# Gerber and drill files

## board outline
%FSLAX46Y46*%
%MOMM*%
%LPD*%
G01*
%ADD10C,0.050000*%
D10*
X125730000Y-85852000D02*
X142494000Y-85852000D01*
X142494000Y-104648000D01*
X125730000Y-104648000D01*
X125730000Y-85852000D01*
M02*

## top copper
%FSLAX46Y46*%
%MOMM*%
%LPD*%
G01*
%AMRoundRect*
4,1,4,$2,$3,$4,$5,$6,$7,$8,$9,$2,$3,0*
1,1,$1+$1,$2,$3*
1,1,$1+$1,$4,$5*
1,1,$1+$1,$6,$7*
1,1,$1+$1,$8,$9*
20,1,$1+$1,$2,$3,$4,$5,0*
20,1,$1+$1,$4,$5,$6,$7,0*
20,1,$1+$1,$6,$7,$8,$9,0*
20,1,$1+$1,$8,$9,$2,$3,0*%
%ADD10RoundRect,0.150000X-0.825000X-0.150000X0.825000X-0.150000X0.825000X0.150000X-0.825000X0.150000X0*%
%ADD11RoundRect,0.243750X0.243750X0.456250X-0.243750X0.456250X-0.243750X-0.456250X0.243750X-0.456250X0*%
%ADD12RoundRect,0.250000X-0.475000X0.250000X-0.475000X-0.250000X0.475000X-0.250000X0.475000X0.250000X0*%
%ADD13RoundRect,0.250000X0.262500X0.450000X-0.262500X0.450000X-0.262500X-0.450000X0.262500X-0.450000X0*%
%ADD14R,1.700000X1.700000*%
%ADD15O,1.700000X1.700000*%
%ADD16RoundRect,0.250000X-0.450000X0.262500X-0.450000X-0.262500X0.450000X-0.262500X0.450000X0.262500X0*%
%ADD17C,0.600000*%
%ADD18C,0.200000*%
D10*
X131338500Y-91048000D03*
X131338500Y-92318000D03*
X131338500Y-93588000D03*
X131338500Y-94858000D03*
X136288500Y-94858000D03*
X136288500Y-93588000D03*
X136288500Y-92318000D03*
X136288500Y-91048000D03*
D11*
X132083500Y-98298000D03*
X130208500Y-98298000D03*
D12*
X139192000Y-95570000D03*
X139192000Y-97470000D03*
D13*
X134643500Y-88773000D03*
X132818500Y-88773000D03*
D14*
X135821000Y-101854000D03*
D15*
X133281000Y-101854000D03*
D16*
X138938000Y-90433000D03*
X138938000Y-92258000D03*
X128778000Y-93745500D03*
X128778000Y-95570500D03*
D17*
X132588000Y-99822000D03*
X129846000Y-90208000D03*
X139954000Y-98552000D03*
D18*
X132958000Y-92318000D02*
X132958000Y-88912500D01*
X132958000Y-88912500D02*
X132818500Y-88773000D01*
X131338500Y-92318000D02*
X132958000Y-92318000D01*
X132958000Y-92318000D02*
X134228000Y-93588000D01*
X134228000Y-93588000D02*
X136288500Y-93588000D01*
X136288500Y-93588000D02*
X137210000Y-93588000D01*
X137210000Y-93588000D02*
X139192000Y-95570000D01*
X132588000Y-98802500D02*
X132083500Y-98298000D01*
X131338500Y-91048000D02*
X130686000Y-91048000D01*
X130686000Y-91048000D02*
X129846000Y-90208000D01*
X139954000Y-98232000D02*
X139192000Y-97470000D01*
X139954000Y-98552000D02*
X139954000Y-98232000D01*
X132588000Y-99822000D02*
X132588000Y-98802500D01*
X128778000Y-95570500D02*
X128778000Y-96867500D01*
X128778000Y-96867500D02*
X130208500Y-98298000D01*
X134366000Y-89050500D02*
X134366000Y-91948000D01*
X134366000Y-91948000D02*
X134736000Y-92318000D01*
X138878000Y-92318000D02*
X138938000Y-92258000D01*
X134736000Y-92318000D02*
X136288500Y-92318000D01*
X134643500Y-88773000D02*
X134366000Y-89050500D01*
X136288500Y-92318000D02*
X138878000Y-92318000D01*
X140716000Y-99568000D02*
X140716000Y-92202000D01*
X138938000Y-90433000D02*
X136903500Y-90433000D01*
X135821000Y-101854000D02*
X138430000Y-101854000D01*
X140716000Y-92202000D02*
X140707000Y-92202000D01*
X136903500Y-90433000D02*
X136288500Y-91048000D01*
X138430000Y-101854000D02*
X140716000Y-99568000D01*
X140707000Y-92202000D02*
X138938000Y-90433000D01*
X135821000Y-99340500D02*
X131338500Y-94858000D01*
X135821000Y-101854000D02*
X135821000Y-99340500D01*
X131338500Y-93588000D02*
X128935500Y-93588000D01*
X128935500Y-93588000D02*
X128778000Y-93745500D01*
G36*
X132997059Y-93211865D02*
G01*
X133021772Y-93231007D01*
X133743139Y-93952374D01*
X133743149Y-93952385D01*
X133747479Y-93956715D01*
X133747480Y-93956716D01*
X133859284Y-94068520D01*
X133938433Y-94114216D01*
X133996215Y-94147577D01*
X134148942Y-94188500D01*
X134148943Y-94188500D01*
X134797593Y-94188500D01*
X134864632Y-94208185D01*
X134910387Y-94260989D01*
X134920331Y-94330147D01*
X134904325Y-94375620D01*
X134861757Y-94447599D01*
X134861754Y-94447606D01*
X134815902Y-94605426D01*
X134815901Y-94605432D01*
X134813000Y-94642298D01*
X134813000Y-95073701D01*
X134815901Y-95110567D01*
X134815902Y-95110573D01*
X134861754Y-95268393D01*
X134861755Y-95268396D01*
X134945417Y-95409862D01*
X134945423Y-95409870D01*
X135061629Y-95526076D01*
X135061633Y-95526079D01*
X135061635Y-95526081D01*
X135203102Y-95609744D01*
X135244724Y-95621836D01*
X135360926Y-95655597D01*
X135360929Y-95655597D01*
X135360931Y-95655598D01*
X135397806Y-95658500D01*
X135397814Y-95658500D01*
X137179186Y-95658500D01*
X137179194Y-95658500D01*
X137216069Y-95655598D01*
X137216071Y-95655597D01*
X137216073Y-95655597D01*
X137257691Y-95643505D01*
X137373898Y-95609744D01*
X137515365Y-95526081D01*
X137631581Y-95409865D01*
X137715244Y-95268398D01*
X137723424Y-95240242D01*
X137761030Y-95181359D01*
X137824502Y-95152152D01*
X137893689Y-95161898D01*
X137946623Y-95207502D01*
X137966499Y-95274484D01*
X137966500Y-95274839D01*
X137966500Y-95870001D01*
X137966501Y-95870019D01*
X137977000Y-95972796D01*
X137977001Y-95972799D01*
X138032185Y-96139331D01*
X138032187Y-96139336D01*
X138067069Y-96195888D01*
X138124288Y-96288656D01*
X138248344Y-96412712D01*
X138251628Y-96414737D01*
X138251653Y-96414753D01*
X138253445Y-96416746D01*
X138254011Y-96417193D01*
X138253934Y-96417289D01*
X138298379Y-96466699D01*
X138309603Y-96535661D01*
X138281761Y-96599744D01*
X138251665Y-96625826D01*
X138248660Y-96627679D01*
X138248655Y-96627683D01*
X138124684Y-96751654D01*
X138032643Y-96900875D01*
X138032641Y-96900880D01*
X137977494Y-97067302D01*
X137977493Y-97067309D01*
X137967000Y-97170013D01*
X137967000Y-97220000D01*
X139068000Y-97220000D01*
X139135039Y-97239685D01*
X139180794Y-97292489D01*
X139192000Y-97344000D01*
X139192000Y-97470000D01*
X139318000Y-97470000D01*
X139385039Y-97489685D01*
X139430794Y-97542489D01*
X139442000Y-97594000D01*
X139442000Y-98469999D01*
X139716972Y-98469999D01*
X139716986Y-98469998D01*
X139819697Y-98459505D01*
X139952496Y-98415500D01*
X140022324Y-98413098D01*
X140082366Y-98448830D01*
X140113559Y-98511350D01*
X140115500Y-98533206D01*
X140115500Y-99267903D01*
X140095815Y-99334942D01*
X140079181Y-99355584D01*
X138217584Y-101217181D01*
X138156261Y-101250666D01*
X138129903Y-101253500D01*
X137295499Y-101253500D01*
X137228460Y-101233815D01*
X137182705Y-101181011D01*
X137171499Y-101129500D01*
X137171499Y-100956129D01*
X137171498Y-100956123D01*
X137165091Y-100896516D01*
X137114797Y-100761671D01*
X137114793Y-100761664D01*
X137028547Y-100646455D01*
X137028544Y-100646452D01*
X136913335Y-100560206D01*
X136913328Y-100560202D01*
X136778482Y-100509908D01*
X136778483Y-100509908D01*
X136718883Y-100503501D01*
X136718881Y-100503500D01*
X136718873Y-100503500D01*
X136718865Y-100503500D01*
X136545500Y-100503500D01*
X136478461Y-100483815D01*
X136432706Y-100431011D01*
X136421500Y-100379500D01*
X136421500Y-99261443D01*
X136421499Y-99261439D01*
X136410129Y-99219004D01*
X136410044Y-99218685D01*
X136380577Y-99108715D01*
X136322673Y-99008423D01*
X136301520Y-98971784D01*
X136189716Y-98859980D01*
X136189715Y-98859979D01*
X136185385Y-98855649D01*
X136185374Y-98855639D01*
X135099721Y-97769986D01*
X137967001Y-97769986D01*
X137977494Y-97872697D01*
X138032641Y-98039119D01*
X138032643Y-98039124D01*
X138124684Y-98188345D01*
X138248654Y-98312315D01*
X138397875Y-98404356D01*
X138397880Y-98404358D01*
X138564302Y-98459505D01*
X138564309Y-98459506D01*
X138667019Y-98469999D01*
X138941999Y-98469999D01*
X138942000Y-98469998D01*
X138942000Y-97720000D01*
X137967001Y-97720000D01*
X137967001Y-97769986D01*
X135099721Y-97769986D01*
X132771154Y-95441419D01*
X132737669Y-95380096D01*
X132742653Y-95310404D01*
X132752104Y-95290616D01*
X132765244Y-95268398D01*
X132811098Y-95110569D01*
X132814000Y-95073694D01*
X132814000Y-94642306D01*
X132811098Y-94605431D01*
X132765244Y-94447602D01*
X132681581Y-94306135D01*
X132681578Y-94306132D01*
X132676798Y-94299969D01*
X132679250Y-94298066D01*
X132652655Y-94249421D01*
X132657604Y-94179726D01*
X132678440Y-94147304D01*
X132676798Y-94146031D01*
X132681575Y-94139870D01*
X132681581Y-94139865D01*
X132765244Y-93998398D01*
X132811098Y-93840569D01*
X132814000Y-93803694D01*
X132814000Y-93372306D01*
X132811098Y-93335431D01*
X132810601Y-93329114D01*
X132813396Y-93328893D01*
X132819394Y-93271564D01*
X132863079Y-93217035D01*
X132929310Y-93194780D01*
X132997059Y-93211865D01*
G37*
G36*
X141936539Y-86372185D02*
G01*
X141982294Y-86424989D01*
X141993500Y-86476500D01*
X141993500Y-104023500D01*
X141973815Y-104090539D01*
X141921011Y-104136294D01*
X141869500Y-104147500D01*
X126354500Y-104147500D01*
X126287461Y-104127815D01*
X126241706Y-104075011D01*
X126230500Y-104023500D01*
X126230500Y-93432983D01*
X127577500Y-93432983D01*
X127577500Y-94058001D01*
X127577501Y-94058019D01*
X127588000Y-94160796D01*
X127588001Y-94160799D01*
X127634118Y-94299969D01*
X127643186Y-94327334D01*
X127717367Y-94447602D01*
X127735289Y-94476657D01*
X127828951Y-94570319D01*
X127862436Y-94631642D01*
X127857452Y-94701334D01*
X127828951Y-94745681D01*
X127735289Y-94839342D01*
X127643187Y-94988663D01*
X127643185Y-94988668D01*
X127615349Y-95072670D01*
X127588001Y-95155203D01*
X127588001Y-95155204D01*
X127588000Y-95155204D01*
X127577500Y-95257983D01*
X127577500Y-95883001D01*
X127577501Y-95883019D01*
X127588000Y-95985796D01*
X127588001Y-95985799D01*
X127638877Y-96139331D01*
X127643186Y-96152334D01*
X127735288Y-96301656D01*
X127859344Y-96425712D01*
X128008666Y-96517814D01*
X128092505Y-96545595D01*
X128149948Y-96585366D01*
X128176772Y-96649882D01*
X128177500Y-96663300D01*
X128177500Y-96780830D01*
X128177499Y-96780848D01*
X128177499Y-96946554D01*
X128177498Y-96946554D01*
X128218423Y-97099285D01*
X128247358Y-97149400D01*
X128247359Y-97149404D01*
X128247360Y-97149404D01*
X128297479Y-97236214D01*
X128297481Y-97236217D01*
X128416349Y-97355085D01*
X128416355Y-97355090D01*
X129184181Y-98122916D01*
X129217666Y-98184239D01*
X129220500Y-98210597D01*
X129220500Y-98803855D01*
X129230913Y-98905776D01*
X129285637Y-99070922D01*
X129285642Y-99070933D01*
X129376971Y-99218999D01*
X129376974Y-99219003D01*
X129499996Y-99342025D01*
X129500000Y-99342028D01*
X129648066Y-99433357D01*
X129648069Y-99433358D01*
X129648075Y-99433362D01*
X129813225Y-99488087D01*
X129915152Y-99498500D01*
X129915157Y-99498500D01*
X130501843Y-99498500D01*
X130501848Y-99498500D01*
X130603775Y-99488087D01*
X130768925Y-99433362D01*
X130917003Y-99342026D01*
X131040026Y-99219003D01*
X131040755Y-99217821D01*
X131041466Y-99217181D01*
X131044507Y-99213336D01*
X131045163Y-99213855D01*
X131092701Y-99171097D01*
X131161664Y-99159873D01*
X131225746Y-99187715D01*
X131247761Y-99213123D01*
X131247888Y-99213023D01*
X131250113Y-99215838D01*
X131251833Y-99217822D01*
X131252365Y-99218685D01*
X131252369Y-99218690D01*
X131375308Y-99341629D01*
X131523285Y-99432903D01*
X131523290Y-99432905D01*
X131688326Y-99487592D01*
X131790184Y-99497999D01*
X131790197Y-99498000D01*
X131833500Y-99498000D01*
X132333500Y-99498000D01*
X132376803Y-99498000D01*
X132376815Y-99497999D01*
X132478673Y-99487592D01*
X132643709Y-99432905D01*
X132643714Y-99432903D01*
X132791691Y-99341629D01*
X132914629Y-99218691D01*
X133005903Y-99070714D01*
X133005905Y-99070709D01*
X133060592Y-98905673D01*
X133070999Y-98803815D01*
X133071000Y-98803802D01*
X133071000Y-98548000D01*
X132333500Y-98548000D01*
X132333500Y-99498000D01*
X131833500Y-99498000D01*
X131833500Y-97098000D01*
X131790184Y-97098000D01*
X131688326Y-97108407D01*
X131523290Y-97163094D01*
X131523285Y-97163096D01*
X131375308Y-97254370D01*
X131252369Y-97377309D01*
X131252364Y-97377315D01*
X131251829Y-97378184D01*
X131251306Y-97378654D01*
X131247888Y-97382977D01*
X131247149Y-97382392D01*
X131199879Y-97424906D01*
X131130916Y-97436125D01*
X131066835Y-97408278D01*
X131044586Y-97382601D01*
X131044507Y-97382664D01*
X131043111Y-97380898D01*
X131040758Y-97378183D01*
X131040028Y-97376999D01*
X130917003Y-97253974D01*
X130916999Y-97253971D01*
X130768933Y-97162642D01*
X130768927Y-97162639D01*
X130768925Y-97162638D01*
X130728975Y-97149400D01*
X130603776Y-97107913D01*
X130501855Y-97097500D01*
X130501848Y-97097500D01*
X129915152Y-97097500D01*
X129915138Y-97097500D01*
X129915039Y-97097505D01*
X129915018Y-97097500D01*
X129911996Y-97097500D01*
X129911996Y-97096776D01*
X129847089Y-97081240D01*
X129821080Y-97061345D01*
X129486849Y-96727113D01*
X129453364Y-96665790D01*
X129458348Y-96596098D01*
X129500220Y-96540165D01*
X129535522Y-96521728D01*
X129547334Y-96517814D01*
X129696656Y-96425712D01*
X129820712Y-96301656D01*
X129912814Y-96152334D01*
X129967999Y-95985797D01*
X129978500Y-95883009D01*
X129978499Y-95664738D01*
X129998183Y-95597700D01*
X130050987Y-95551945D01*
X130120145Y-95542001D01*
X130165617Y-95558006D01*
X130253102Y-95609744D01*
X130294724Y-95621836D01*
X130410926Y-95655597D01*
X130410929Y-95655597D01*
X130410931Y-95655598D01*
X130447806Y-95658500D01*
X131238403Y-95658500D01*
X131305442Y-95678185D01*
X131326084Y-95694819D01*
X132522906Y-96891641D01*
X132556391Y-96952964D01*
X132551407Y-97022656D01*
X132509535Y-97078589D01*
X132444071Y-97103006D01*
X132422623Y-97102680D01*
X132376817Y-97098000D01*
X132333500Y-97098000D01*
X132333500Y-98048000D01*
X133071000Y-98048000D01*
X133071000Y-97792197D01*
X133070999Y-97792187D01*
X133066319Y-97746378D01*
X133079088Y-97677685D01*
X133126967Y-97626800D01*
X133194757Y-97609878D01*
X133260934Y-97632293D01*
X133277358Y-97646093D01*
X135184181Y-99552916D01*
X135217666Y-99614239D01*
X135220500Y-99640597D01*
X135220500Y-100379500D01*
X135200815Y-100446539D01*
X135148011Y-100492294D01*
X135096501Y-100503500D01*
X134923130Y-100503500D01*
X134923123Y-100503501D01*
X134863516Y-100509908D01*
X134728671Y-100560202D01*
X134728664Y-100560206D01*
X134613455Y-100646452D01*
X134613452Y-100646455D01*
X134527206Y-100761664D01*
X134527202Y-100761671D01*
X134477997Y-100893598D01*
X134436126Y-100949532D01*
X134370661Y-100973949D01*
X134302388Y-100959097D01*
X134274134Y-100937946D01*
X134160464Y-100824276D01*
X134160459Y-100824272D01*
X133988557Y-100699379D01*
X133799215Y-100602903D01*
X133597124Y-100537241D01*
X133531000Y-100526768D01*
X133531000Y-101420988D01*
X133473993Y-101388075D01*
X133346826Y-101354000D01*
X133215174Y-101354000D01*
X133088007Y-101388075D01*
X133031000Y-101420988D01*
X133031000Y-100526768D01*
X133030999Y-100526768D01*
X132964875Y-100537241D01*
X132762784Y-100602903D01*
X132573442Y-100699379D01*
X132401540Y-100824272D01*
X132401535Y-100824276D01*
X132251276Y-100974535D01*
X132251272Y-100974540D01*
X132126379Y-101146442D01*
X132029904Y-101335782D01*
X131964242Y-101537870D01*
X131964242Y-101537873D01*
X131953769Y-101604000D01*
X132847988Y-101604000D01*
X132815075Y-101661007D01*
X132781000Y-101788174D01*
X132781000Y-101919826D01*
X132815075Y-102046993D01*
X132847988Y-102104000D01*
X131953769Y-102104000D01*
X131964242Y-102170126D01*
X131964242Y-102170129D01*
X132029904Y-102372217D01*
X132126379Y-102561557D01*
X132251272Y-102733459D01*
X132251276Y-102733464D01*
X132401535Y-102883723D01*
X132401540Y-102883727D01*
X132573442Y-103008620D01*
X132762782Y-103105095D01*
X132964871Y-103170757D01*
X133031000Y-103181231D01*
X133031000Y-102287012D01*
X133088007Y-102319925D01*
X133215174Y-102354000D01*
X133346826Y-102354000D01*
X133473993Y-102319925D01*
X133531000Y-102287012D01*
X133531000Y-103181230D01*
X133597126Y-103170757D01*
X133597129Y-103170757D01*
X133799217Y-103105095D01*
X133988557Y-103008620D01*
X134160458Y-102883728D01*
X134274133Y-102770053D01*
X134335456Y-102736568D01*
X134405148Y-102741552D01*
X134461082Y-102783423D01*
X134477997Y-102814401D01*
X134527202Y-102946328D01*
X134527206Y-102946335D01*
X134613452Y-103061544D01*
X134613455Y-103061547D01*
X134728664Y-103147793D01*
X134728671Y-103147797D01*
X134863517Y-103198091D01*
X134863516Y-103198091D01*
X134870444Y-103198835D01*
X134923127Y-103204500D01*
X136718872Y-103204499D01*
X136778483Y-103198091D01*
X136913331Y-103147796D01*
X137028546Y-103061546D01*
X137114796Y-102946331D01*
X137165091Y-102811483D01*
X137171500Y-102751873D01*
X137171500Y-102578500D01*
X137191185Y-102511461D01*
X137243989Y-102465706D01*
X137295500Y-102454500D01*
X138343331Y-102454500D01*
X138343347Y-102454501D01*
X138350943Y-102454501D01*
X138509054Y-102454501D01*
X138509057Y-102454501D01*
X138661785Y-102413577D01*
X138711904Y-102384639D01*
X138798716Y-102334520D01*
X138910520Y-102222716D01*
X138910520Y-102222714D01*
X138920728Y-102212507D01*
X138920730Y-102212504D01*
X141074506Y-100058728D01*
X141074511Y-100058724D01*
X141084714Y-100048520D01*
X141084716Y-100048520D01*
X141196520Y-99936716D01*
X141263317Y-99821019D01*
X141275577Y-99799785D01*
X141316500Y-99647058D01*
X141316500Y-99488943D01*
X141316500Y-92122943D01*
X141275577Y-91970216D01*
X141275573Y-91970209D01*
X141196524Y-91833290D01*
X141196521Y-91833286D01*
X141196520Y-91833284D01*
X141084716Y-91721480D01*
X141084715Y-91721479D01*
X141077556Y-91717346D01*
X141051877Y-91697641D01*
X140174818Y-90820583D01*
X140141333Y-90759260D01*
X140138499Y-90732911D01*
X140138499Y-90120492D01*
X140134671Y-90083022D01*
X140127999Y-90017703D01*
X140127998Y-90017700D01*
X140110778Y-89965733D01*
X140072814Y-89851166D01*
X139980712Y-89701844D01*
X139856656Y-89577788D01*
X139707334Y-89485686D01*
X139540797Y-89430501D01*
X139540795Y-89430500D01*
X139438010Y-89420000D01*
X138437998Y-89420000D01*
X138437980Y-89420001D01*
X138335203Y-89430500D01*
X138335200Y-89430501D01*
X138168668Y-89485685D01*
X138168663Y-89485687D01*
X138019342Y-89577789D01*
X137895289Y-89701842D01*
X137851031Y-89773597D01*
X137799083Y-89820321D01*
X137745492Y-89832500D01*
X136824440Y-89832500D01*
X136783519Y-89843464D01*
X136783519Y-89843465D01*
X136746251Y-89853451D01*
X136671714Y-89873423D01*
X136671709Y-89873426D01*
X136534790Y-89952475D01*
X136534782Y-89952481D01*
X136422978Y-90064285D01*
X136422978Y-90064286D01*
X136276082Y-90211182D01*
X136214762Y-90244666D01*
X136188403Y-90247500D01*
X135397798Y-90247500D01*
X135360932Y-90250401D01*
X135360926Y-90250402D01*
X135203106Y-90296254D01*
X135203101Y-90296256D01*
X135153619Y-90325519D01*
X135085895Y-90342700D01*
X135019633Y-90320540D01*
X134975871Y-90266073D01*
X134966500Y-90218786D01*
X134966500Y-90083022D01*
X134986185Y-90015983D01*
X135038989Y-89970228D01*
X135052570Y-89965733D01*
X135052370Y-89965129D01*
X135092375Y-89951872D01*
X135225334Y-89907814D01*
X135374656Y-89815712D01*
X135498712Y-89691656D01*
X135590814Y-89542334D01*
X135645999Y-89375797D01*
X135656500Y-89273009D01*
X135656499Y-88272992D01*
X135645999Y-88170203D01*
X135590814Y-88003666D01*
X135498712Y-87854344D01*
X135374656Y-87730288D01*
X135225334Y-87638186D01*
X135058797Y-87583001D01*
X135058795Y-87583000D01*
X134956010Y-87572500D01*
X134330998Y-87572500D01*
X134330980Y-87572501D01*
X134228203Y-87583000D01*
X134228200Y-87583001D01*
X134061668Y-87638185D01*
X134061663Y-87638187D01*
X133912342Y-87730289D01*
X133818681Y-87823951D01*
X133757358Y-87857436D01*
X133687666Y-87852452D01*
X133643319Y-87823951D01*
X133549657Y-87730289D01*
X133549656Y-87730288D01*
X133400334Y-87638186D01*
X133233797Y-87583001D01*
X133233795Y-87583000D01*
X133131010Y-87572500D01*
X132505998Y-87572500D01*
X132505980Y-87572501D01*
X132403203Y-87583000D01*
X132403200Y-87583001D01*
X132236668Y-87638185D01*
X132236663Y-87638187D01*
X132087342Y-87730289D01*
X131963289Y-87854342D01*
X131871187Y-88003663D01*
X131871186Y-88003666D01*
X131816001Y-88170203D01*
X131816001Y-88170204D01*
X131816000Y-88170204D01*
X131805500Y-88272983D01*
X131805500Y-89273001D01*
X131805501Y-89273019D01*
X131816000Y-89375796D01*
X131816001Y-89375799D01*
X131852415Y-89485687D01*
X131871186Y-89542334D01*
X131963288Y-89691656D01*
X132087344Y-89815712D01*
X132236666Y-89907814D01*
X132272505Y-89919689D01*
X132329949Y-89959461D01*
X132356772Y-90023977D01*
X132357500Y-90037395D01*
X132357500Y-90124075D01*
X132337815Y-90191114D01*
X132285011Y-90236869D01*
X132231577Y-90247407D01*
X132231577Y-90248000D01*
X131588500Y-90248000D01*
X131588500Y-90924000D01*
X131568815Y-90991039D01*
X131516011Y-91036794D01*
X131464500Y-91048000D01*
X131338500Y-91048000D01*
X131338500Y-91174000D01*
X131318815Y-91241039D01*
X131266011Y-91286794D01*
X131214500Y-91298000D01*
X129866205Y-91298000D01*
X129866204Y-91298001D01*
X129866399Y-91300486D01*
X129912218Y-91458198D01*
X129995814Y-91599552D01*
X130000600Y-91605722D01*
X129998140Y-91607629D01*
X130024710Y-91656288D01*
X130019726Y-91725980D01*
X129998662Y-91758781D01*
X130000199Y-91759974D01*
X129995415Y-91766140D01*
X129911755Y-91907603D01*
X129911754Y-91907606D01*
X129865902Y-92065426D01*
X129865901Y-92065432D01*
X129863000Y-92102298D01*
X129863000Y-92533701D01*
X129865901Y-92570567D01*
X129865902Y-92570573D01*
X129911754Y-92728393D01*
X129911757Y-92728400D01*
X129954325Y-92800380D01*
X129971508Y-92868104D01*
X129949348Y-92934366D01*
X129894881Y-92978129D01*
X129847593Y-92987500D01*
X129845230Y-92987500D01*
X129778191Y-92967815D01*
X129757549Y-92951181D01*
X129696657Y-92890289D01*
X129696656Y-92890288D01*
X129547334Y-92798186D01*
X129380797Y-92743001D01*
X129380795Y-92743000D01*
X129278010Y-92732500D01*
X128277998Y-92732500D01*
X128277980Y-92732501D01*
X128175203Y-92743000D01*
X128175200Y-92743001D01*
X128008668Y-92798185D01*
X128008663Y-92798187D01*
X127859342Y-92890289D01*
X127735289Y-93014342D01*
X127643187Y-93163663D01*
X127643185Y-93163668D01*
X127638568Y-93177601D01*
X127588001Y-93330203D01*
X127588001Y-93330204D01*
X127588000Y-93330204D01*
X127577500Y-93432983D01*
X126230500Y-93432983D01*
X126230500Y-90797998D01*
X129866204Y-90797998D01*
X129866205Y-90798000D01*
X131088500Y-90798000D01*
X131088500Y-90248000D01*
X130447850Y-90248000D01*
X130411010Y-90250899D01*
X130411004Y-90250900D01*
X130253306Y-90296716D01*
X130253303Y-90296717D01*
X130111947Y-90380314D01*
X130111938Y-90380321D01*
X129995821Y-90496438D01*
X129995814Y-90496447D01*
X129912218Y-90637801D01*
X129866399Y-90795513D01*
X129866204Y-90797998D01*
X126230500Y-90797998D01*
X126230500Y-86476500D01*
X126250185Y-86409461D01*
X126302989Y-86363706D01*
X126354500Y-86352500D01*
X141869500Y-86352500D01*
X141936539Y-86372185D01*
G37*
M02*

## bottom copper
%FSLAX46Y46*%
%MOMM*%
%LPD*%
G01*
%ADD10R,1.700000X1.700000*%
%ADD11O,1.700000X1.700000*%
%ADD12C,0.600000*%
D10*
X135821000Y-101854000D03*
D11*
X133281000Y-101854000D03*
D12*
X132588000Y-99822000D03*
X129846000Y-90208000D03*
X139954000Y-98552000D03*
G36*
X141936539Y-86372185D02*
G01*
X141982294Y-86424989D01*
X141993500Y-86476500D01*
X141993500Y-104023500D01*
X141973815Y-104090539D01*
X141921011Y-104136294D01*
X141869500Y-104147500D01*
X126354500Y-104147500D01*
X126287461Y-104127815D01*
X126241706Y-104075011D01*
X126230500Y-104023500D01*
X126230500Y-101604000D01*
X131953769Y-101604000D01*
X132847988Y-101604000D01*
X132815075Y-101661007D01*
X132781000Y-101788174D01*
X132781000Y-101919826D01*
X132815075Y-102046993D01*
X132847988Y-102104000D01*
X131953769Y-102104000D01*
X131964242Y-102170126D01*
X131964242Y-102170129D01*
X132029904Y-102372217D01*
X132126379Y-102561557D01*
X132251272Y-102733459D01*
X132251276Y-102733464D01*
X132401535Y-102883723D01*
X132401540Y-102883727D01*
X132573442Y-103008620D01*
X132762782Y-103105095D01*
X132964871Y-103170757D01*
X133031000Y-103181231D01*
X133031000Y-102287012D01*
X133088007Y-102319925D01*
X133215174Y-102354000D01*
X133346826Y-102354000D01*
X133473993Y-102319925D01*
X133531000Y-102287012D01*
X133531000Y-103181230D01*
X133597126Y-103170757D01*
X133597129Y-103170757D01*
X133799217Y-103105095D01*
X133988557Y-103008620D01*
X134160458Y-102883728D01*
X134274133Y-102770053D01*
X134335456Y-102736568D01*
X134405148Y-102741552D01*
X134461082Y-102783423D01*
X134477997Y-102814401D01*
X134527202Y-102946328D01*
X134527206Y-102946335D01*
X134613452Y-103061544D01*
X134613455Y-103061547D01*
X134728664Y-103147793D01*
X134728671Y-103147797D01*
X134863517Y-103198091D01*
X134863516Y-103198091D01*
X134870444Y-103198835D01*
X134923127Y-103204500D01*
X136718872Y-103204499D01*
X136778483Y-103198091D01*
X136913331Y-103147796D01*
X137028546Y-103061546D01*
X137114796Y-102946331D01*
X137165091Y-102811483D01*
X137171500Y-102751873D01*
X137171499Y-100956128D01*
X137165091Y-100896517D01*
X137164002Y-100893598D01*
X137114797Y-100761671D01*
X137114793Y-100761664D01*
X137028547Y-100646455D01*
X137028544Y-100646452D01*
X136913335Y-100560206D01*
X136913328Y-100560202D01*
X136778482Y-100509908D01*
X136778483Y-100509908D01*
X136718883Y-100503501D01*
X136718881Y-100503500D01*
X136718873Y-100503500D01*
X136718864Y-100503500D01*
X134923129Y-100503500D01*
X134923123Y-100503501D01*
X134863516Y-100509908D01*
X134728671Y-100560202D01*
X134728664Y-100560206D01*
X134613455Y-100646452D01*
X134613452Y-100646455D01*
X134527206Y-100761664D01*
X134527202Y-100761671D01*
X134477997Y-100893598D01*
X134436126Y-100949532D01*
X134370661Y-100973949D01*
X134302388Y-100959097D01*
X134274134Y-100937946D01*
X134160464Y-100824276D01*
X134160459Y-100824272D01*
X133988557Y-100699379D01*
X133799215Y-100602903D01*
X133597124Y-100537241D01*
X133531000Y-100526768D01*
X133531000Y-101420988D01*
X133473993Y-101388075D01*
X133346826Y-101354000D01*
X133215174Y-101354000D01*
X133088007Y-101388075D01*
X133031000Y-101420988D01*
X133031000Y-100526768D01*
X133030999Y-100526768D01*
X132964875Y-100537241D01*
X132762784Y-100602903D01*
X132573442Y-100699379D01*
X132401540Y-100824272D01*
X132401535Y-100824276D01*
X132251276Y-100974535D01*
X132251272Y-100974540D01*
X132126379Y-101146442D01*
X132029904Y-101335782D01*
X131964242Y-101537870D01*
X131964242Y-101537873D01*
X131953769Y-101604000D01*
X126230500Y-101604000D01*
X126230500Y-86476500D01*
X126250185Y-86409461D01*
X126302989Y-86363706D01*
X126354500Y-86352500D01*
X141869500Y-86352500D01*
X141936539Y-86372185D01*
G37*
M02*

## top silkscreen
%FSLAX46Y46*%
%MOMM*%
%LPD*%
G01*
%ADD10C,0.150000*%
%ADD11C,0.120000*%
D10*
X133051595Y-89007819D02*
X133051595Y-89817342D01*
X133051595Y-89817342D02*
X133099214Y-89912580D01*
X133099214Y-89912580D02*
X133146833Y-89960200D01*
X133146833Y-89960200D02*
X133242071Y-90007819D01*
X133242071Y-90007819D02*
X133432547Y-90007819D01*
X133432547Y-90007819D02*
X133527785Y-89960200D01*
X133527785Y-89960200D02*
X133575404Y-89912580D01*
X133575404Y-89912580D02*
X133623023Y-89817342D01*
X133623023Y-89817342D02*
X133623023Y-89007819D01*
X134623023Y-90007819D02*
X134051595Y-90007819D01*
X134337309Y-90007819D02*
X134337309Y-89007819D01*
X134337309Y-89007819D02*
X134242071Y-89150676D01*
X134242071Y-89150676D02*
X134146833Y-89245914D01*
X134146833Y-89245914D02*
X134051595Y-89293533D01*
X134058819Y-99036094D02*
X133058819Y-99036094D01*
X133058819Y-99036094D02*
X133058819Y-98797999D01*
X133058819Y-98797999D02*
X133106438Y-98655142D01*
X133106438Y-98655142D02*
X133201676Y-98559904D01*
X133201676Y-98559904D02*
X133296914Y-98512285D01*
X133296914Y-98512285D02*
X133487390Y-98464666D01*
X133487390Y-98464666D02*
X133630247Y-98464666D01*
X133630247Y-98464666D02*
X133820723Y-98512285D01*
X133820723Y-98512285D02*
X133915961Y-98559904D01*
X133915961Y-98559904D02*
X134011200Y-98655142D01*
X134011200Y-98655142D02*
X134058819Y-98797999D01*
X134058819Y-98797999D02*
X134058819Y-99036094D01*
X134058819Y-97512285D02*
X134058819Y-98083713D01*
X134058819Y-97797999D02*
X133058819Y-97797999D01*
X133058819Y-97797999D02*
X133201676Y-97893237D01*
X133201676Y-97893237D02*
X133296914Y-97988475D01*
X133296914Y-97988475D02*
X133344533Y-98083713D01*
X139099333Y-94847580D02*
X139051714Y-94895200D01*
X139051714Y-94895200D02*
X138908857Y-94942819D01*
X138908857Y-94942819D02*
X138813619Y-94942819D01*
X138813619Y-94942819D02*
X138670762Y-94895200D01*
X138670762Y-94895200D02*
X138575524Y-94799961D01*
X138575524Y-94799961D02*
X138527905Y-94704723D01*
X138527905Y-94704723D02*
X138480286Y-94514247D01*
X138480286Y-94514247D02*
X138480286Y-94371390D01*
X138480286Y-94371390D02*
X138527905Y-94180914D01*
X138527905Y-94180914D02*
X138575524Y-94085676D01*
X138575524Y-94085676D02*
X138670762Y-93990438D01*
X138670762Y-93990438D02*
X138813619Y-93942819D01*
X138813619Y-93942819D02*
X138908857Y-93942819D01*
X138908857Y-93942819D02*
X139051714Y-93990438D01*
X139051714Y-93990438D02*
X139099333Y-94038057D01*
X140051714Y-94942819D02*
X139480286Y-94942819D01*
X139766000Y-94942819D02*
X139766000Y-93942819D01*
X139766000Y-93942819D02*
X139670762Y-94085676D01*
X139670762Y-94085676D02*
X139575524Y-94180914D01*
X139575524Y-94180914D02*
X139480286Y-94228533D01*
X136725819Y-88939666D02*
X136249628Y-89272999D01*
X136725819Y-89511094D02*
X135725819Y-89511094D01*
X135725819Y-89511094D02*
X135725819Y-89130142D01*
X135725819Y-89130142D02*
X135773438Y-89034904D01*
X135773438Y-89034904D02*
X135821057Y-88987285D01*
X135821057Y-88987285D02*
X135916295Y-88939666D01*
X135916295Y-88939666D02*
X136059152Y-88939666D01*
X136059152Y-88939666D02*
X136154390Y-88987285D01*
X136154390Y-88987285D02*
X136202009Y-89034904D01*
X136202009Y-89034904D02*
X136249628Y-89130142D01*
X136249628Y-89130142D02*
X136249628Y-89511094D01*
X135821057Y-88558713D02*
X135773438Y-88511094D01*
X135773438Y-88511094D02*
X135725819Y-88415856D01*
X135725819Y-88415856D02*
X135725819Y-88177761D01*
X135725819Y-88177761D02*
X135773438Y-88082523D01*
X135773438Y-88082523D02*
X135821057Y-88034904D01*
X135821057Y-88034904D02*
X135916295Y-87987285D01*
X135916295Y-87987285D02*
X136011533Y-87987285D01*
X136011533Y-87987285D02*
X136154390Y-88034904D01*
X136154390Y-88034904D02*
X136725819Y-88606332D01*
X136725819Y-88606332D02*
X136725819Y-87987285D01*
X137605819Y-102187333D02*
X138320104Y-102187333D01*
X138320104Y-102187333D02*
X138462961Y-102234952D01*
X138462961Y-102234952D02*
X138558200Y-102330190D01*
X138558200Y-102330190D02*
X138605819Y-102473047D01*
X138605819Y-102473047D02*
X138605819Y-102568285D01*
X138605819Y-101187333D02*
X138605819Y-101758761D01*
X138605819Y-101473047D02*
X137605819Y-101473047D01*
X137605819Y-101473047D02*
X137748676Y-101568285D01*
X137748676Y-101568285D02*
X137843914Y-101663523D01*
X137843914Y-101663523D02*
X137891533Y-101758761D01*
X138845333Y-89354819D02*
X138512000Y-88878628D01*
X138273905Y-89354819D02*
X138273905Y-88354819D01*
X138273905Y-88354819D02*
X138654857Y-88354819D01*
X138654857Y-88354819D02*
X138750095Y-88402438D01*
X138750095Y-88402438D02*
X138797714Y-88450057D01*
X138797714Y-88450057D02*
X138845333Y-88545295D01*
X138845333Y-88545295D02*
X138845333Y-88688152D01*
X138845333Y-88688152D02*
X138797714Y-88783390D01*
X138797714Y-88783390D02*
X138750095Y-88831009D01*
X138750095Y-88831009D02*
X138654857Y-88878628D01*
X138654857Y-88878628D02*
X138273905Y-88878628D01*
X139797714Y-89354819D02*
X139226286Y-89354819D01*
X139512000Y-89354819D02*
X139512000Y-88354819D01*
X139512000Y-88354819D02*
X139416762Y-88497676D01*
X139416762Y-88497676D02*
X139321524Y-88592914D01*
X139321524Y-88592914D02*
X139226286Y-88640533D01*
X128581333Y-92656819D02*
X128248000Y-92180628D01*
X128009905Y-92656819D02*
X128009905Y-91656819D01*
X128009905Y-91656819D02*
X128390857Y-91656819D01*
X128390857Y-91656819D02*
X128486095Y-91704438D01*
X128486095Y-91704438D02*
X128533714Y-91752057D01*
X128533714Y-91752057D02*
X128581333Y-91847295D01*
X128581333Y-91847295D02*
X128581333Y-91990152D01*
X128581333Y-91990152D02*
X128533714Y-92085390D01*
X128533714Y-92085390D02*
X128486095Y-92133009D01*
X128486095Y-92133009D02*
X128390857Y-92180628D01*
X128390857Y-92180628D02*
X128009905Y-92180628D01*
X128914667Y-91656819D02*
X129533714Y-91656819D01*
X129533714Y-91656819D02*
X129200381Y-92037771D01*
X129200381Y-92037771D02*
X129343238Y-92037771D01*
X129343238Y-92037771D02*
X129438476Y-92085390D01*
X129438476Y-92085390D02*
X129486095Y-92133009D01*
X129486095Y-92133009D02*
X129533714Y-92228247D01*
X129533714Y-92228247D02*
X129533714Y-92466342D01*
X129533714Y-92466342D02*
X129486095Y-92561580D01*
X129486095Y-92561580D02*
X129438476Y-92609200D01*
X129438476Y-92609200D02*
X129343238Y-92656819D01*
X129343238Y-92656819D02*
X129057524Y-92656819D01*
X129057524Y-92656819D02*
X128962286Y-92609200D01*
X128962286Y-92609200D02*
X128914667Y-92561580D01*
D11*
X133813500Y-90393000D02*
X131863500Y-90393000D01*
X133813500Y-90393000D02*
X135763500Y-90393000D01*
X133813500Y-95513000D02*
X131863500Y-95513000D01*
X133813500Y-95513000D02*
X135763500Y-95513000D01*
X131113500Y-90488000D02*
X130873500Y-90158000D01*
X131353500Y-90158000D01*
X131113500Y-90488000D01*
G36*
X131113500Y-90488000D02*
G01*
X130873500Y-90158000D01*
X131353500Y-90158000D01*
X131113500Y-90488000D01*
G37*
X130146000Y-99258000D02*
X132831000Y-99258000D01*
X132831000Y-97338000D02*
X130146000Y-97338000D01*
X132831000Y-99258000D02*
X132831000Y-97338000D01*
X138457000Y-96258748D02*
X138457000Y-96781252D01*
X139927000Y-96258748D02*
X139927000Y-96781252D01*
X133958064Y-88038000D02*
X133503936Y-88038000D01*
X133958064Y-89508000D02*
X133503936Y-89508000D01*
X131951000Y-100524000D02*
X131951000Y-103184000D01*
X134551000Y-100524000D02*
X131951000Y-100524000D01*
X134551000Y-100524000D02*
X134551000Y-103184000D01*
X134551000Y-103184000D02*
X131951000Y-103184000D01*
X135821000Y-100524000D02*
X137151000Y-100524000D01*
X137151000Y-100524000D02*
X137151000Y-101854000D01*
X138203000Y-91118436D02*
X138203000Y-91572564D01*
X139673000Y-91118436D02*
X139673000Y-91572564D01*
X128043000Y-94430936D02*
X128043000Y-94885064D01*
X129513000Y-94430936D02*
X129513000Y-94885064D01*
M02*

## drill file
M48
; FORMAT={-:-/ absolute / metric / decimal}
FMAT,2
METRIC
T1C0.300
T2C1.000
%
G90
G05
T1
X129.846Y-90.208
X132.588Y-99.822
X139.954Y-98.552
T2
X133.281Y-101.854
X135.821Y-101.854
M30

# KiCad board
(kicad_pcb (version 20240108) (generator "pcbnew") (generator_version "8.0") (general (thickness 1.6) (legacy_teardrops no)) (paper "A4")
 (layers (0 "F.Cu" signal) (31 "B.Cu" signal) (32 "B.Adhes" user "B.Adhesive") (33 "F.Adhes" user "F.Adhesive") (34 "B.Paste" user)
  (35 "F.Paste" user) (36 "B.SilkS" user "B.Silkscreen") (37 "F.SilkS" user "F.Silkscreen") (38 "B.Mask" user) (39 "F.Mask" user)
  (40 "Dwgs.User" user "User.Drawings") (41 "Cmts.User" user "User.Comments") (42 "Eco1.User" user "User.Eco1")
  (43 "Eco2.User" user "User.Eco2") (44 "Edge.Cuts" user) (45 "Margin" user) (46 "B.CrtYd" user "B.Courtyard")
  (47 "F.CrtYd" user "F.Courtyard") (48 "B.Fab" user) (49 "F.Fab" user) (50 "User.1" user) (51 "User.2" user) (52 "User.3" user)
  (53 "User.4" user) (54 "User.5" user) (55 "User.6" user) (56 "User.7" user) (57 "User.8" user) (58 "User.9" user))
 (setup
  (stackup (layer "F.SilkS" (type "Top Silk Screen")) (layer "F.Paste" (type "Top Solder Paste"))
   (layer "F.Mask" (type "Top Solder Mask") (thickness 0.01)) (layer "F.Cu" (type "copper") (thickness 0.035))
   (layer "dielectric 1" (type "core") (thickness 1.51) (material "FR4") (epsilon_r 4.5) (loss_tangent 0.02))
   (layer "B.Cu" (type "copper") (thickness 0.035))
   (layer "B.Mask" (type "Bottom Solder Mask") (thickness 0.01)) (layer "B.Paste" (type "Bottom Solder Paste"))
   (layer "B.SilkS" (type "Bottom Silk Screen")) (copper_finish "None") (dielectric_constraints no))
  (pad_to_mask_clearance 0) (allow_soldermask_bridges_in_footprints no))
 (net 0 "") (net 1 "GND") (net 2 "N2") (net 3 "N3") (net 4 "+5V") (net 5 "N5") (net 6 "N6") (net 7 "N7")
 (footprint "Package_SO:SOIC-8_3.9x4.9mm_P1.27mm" (layer "F.Cu") (at 133.8135 92.953)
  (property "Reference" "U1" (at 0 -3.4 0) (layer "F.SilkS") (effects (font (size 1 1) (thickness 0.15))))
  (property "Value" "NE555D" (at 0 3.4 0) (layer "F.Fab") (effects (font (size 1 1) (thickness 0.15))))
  (fp_line (start 0 -2.56) (end -1.95 -2.56) (stroke (width 0.12) (type solid)) (layer "F.SilkS"))
  (fp_line (start 0 -2.56) (end 1.95 -2.56) (stroke (width 0.12) (type solid)) (layer "F.SilkS"))
  (fp_line (start 0 2.56) (end -1.95 2.56) (stroke (width 0.12) (type solid)) (layer "F.SilkS"))
  (fp_line (start 0 2.56) (end 1.95 2.56) (stroke (width 0.12) (type solid)) (layer "F.SilkS"))
  (fp_poly
   (pts (xy -2.7 -2.465) (xy -2.94 -2.795) (xy -2.46 -2.795) (xy -2.7 -2.465)) (stroke (width 0.12) (type solid)) (fill solid)
   (layer "F.SilkS"))
  (pad "1" smd roundrect (at -2.475 -1.905) (size 1.95 0.6) (layers "F.Cu" "F.Paste" "F.Mask") (roundrect_rratio 0.25) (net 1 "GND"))
  (pad "2" smd roundrect (at -2.475 -0.635) (size 1.95 0.6) (layers "F.Cu" "F.Paste" "F.Mask") (roundrect_rratio 0.25) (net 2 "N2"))
  (pad "3" smd roundrect (at -2.475 0.635) (size 1.95 0.6) (layers "F.Cu" "F.Paste" "F.Mask") (roundrect_rratio 0.25) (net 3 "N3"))
  (pad "4" smd roundrect (at -2.475 1.905) (size 1.95 0.6) (layers "F.Cu" "F.Paste" "F.Mask") (roundrect_rratio 0.25) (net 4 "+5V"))
  (pad "5" smd roundrect (at 2.475 1.905) (size 1.95 0.6) (layers "F.Cu" "F.Paste" "F.Mask") (roundrect_rratio 0.25) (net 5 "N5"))
  (pad "6" smd roundrect (at 2.475 0.635) (size 1.95 0.6) (layers "F.Cu" "F.Paste" "F.Mask") (roundrect_rratio 0.25) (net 2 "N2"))
  (pad "7" smd roundrect (at 2.475 -0.635) (size 1.95 0.6) (layers "F.Cu" "F.Paste" "F.Mask") (roundrect_rratio 0.25) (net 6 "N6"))
  (pad "8" smd roundrect (at 2.475 -1.905) (size 1.95 0.6) (layers "F.Cu" "F.Paste" "F.Mask") (roundrect_rratio 0.25) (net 4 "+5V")))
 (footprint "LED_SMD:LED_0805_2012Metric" (layer "F.Cu") (at 131.146 98.298 180)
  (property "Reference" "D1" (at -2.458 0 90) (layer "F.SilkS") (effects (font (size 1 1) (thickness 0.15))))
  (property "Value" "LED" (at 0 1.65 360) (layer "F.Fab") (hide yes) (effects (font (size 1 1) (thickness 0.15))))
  (fp_line (start 1 -0.96) (end -1.685 -0.96) (stroke (width 0.12) (type solid)) (layer "F.SilkS"))
  (fp_line (start -1.685 0.96) (end 1 0.96) (stroke (width 0.12) (type solid)) (layer "F.SilkS"))
  (fp_line (start -1.685 -0.96) (end -1.685 0.96) (stroke (width 0.12) (type solid)) (layer "F.SilkS"))
  (pad "1" smd roundrect (at -0.9375 0 180) (size 0.975 1.4) (layers "F.Cu" "F.Paste" "F.Mask") (roundrect_rratio 0.25) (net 1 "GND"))
  (pad "2" smd roundrect (at 0.9375 0 180) (size 0.975 1.4) (layers "F.Cu" "F.Paste" "F.Mask") (roundrect_rratio 0.25) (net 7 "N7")))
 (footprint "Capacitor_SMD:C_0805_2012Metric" (layer "F.Cu") (at 139.192 96.52 -90)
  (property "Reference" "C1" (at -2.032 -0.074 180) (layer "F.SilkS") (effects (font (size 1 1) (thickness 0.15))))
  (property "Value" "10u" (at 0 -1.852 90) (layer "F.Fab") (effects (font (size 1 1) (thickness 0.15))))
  (fp_line (start -0.261252 0.735) (end 0.261252 0.735) (stroke (width 0.12) (type solid)) (layer "F.SilkS"))
  (fp_line (start -0.261252 -0.735) (end 0.261252 -0.735) (stroke (width 0.12) (type solid)) (layer "F.SilkS"))
  (pad "1" smd roundrect (at -0.95 0 270) (size 1 1.45) (layers "F.Cu" "F.Paste" "F.Mask") (roundrect_rratio 0.25) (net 2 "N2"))
  (pad "2" smd roundrect (at 0.95 0 270) (size 1 1.45) (layers "F.Cu" "F.Paste" "F.Mask") (roundrect_rratio 0.25) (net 1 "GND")))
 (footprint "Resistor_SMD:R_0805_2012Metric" (layer "F.Cu") (at 133.731 88.773 180)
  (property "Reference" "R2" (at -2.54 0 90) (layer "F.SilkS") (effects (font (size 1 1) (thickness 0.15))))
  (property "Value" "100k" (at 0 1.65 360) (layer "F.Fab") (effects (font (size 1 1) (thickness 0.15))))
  (fp_line (start -0.227064 0.735) (end 0.227064 0.735) (stroke (width 0.12) (type solid)) (layer "F.SilkS"))
  (fp_line (start -0.227064 -0.735) (end 0.227064 -0.735) (stroke (width 0.12) (type solid)) (layer "F.SilkS"))
  (pad "1" smd roundrect (at -0.9125 0 180) (size 1.025 1.4) (layers "F.Cu" "F.Paste" "F.Mask") (roundrect_rratio 0.243902) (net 6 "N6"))
  (pad "2" smd roundrect (at 0.9125 0 180) (size 1.025 1.4) (layers "F.Cu" "F.Paste" "F.Mask") (roundrect_rratio 0.243902) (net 2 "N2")))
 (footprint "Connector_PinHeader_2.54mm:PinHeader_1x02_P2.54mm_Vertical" (layer "F.Cu") (at 135.821 101.854 -90)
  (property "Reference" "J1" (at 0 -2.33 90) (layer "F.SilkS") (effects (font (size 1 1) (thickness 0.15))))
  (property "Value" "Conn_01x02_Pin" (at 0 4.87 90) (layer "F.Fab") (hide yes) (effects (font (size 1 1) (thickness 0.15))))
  (fp_line (start -1.33 3.87) (end 1.33 3.87) (stroke (width 0.12) (type solid)) (layer "F.SilkS"))
  (fp_line (start -1.33 1.27) (end -1.33 3.87) (stroke (width 0.12) (type solid)) (layer "F.SilkS"))
  (fp_line (start -1.33 1.27) (end 1.33 1.27) (stroke (width 0.12) (type solid)) (layer "F.SilkS"))
  (fp_line (start 1.33 1.27) (end 1.33 3.87) (stroke (width 0.12) (type solid)) (layer "F.SilkS"))
  (fp_line (start -1.33 0) (end -1.33 -1.33) (stroke (width 0.12) (type solid)) (layer "F.SilkS"))
  (fp_line (start -1.33 -1.33) (end 0 -1.33) (stroke (width 0.12) (type solid)) (layer "F.SilkS"))
  (pad "1" thru_hole rect (at 0 0 270) (size 1.7 1.7) (drill 1) (layers "*.Cu" "*.Mask") (remove_unused_layers no) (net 4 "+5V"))
  (pad "2" thru_hole oval (at 0 2.54 270) (size 1.7 1.7) (drill 1) (layers "*.Cu" "*.Mask") (remove_unused_layers no) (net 1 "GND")))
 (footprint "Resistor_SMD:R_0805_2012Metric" (layer "F.Cu") (at 138.938 91.3455 -90)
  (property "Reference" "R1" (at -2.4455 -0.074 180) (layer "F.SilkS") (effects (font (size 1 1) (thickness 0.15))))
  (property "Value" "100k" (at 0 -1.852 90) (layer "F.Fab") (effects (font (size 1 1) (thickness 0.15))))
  (fp_line (start -0.227064 0.735) (end 0.227064 0.735) (stroke (width 0.12) (type solid)) (layer "F.SilkS"))
  (fp_line (start -0.227064 -0.735) (end 0.227064 -0.735) (stroke (width 0.12) (type solid)) (layer "F.SilkS"))
  (pad "1" smd roundrect (at -0.9125 0 270) (size 1.025 1.4) (layers "F.Cu" "F.Paste" "F.Mask") (roundrect_rratio 0.243902) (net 4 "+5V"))
  (pad "2" smd roundrect (at 0.9125 0 270) (size 1.025 1.4) (layers "F.Cu" "F.Paste" "F.Mask") (roundrect_rratio 0.243902) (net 6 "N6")))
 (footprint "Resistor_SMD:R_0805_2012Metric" (layer "F.Cu") (at 128.778 94.658 -90)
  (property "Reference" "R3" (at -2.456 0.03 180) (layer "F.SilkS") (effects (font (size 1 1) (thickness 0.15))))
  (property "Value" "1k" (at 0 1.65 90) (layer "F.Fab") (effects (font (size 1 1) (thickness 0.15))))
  (fp_line (start -0.227064 0.735) (end 0.227064 0.735) (stroke (width 0.12) (type solid)) (layer "F.SilkS"))
  (fp_line (start -0.227064 -0.735) (end 0.227064 -0.735) (stroke (width 0.12) (type solid)) (layer "F.SilkS"))
  (pad "1" smd roundrect (at -0.9125 0 270) (size 1.025 1.4) (layers "F.Cu" "F.Paste" "F.Mask") (roundrect_rratio 0.243902) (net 3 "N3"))
  (pad "2" smd roundrect (at 0.9125 0 270) (size 1.025 1.4) (layers "F.Cu" "F.Paste" "F.Mask") (roundrect_rratio 0.243902) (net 7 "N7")))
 (gr_rect (start 125.73 85.852) (end 142.494 104.648) (stroke (width 0.05) (type default)) (fill none) (layer "Edge.Cuts"))
 (segment (start 132.958 92.318) (end 132.958 88.9125) (width 0.2) (layer "F.Cu") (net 2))
 (segment (start 132.958 88.9125) (end 132.8185 88.773) (width 0.2) (layer "F.Cu") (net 2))
 (segment (start 131.3385 92.318) (end 132.958 92.318) (width 0.2) (layer "F.Cu") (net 2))
 (segment (start 132.958 92.318) (end 134.228 93.588) (width 0.2) (layer "F.Cu") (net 2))
 (segment (start 134.228 93.588) (end 136.2885 93.588) (width 0.2) (layer "F.Cu") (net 2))
 (segment (start 136.2885 93.588) (end 137.21 93.588) (width 0.2) (layer "F.Cu") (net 2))
 (segment (start 137.21 93.588) (end 139.192 95.57) (width 0.2) (layer "F.Cu") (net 2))
 (segment (start 132.588 98.8025) (end 132.0835 98.298) (width 0.2) (layer "F.Cu") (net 1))
 (segment (start 131.3385 91.048) (end 130.686 91.048) (width 0.2) (layer "F.Cu") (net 1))
 (segment (start 130.686 91.048) (end 129.846 90.208) (width 0.2) (layer "F.Cu") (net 1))
 (segment (start 139.954 98.232) (end 139.192 97.47) (width 0.2) (layer "F.Cu") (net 1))
 (segment (start 139.954 98.552) (end 139.954 98.232) (width 0.2) (layer "F.Cu") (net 1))
 (segment (start 132.588 99.822) (end 132.588 98.8025) (width 0.2) (layer "F.Cu") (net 1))
 (via (at 132.588 99.822) (size 0.6) (drill 0.3) (layers "F.Cu" "B.Cu") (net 1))
 (via (at 129.846 90.208) (size 0.6) (drill 0.3) (layers "F.Cu" "B.Cu") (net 1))
 (via (at 139.954 98.552) (size 0.6) (drill 0.3) (layers "F.Cu" "B.Cu") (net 1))
 (segment (start 128.778 95.5705) (end 128.778 96.8675) (width 0.2) (layer "F.Cu") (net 7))
 (segment (start 128.778 96.8675) (end 130.2085 98.298) (width 0.2) (layer "F.Cu") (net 7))
 (segment (start 134.366 89.0505) (end 134.366 91.948) (width 0.2) (layer "F.Cu") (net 6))
 (segment (start 134.366 91.948) (end 134.736 92.318) (width 0.2) (layer "F.Cu") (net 6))
 (segment (start 138.878 92.318) (end 138.938 92.258) (width 0.2) (layer "F.Cu") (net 6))
 (segment (start 134.736 92.318) (end 136.2885 92.318) (width 0.2) (layer "F.Cu") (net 6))
 (segment (start 134.6435 88.773) (end 134.366 89.0505) (width 0.2) (layer "F.Cu") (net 6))
 (segment (start 136.2885 92.318) (end 138.878 92.318) (width 0.2) (layer "F.Cu") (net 6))
 (segment (start 140.716 99.568) (end 140.716 92.202) (width 0.2) (layer "F.Cu") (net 4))
 (segment (start 138.938 90.433) (end 136.9035 90.433) (width 0.2) (layer "F.Cu") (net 4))
 (segment (start 135.821 101.854) (end 138.43 101.854) (width 0.2) (layer "F.Cu") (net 4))
 (segment (start 140.716 92.202) (end 140.707 92.202) (width 0.2) (layer "F.Cu") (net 4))
 (segment (start 136.9035 90.433) (end 136.2885 91.048) (width 0.2) (layer "F.Cu") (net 4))
 (segment (start 138.43 101.854) (end 140.716 99.568) (width 0.2) (layer "F.Cu") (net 4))
 (segment (start 140.707 92.202) (end 138.938 90.433) (width 0.2) (layer "F.Cu") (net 4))
 (segment (start 135.821 99.3405) (end 131.3385 94.858) (width 0.2) (layer "F.Cu") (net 4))
 (segment (start 135.821 101.854) (end 135.821 99.3405) (width 0.2) (layer "F.Cu") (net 4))
 (segment (start 131.3385 93.588) (end 128.9355 93.588) (width 0.2) (layer "F.Cu") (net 3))
 (segment (start 128.9355 93.588) (end 128.778 93.7455) (width 0.2) (layer "F.Cu") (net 3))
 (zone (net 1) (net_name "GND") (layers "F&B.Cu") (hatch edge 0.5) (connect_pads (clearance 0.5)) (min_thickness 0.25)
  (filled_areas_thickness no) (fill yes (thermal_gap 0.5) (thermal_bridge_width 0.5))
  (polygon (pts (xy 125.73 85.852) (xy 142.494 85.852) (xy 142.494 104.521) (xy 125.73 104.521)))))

